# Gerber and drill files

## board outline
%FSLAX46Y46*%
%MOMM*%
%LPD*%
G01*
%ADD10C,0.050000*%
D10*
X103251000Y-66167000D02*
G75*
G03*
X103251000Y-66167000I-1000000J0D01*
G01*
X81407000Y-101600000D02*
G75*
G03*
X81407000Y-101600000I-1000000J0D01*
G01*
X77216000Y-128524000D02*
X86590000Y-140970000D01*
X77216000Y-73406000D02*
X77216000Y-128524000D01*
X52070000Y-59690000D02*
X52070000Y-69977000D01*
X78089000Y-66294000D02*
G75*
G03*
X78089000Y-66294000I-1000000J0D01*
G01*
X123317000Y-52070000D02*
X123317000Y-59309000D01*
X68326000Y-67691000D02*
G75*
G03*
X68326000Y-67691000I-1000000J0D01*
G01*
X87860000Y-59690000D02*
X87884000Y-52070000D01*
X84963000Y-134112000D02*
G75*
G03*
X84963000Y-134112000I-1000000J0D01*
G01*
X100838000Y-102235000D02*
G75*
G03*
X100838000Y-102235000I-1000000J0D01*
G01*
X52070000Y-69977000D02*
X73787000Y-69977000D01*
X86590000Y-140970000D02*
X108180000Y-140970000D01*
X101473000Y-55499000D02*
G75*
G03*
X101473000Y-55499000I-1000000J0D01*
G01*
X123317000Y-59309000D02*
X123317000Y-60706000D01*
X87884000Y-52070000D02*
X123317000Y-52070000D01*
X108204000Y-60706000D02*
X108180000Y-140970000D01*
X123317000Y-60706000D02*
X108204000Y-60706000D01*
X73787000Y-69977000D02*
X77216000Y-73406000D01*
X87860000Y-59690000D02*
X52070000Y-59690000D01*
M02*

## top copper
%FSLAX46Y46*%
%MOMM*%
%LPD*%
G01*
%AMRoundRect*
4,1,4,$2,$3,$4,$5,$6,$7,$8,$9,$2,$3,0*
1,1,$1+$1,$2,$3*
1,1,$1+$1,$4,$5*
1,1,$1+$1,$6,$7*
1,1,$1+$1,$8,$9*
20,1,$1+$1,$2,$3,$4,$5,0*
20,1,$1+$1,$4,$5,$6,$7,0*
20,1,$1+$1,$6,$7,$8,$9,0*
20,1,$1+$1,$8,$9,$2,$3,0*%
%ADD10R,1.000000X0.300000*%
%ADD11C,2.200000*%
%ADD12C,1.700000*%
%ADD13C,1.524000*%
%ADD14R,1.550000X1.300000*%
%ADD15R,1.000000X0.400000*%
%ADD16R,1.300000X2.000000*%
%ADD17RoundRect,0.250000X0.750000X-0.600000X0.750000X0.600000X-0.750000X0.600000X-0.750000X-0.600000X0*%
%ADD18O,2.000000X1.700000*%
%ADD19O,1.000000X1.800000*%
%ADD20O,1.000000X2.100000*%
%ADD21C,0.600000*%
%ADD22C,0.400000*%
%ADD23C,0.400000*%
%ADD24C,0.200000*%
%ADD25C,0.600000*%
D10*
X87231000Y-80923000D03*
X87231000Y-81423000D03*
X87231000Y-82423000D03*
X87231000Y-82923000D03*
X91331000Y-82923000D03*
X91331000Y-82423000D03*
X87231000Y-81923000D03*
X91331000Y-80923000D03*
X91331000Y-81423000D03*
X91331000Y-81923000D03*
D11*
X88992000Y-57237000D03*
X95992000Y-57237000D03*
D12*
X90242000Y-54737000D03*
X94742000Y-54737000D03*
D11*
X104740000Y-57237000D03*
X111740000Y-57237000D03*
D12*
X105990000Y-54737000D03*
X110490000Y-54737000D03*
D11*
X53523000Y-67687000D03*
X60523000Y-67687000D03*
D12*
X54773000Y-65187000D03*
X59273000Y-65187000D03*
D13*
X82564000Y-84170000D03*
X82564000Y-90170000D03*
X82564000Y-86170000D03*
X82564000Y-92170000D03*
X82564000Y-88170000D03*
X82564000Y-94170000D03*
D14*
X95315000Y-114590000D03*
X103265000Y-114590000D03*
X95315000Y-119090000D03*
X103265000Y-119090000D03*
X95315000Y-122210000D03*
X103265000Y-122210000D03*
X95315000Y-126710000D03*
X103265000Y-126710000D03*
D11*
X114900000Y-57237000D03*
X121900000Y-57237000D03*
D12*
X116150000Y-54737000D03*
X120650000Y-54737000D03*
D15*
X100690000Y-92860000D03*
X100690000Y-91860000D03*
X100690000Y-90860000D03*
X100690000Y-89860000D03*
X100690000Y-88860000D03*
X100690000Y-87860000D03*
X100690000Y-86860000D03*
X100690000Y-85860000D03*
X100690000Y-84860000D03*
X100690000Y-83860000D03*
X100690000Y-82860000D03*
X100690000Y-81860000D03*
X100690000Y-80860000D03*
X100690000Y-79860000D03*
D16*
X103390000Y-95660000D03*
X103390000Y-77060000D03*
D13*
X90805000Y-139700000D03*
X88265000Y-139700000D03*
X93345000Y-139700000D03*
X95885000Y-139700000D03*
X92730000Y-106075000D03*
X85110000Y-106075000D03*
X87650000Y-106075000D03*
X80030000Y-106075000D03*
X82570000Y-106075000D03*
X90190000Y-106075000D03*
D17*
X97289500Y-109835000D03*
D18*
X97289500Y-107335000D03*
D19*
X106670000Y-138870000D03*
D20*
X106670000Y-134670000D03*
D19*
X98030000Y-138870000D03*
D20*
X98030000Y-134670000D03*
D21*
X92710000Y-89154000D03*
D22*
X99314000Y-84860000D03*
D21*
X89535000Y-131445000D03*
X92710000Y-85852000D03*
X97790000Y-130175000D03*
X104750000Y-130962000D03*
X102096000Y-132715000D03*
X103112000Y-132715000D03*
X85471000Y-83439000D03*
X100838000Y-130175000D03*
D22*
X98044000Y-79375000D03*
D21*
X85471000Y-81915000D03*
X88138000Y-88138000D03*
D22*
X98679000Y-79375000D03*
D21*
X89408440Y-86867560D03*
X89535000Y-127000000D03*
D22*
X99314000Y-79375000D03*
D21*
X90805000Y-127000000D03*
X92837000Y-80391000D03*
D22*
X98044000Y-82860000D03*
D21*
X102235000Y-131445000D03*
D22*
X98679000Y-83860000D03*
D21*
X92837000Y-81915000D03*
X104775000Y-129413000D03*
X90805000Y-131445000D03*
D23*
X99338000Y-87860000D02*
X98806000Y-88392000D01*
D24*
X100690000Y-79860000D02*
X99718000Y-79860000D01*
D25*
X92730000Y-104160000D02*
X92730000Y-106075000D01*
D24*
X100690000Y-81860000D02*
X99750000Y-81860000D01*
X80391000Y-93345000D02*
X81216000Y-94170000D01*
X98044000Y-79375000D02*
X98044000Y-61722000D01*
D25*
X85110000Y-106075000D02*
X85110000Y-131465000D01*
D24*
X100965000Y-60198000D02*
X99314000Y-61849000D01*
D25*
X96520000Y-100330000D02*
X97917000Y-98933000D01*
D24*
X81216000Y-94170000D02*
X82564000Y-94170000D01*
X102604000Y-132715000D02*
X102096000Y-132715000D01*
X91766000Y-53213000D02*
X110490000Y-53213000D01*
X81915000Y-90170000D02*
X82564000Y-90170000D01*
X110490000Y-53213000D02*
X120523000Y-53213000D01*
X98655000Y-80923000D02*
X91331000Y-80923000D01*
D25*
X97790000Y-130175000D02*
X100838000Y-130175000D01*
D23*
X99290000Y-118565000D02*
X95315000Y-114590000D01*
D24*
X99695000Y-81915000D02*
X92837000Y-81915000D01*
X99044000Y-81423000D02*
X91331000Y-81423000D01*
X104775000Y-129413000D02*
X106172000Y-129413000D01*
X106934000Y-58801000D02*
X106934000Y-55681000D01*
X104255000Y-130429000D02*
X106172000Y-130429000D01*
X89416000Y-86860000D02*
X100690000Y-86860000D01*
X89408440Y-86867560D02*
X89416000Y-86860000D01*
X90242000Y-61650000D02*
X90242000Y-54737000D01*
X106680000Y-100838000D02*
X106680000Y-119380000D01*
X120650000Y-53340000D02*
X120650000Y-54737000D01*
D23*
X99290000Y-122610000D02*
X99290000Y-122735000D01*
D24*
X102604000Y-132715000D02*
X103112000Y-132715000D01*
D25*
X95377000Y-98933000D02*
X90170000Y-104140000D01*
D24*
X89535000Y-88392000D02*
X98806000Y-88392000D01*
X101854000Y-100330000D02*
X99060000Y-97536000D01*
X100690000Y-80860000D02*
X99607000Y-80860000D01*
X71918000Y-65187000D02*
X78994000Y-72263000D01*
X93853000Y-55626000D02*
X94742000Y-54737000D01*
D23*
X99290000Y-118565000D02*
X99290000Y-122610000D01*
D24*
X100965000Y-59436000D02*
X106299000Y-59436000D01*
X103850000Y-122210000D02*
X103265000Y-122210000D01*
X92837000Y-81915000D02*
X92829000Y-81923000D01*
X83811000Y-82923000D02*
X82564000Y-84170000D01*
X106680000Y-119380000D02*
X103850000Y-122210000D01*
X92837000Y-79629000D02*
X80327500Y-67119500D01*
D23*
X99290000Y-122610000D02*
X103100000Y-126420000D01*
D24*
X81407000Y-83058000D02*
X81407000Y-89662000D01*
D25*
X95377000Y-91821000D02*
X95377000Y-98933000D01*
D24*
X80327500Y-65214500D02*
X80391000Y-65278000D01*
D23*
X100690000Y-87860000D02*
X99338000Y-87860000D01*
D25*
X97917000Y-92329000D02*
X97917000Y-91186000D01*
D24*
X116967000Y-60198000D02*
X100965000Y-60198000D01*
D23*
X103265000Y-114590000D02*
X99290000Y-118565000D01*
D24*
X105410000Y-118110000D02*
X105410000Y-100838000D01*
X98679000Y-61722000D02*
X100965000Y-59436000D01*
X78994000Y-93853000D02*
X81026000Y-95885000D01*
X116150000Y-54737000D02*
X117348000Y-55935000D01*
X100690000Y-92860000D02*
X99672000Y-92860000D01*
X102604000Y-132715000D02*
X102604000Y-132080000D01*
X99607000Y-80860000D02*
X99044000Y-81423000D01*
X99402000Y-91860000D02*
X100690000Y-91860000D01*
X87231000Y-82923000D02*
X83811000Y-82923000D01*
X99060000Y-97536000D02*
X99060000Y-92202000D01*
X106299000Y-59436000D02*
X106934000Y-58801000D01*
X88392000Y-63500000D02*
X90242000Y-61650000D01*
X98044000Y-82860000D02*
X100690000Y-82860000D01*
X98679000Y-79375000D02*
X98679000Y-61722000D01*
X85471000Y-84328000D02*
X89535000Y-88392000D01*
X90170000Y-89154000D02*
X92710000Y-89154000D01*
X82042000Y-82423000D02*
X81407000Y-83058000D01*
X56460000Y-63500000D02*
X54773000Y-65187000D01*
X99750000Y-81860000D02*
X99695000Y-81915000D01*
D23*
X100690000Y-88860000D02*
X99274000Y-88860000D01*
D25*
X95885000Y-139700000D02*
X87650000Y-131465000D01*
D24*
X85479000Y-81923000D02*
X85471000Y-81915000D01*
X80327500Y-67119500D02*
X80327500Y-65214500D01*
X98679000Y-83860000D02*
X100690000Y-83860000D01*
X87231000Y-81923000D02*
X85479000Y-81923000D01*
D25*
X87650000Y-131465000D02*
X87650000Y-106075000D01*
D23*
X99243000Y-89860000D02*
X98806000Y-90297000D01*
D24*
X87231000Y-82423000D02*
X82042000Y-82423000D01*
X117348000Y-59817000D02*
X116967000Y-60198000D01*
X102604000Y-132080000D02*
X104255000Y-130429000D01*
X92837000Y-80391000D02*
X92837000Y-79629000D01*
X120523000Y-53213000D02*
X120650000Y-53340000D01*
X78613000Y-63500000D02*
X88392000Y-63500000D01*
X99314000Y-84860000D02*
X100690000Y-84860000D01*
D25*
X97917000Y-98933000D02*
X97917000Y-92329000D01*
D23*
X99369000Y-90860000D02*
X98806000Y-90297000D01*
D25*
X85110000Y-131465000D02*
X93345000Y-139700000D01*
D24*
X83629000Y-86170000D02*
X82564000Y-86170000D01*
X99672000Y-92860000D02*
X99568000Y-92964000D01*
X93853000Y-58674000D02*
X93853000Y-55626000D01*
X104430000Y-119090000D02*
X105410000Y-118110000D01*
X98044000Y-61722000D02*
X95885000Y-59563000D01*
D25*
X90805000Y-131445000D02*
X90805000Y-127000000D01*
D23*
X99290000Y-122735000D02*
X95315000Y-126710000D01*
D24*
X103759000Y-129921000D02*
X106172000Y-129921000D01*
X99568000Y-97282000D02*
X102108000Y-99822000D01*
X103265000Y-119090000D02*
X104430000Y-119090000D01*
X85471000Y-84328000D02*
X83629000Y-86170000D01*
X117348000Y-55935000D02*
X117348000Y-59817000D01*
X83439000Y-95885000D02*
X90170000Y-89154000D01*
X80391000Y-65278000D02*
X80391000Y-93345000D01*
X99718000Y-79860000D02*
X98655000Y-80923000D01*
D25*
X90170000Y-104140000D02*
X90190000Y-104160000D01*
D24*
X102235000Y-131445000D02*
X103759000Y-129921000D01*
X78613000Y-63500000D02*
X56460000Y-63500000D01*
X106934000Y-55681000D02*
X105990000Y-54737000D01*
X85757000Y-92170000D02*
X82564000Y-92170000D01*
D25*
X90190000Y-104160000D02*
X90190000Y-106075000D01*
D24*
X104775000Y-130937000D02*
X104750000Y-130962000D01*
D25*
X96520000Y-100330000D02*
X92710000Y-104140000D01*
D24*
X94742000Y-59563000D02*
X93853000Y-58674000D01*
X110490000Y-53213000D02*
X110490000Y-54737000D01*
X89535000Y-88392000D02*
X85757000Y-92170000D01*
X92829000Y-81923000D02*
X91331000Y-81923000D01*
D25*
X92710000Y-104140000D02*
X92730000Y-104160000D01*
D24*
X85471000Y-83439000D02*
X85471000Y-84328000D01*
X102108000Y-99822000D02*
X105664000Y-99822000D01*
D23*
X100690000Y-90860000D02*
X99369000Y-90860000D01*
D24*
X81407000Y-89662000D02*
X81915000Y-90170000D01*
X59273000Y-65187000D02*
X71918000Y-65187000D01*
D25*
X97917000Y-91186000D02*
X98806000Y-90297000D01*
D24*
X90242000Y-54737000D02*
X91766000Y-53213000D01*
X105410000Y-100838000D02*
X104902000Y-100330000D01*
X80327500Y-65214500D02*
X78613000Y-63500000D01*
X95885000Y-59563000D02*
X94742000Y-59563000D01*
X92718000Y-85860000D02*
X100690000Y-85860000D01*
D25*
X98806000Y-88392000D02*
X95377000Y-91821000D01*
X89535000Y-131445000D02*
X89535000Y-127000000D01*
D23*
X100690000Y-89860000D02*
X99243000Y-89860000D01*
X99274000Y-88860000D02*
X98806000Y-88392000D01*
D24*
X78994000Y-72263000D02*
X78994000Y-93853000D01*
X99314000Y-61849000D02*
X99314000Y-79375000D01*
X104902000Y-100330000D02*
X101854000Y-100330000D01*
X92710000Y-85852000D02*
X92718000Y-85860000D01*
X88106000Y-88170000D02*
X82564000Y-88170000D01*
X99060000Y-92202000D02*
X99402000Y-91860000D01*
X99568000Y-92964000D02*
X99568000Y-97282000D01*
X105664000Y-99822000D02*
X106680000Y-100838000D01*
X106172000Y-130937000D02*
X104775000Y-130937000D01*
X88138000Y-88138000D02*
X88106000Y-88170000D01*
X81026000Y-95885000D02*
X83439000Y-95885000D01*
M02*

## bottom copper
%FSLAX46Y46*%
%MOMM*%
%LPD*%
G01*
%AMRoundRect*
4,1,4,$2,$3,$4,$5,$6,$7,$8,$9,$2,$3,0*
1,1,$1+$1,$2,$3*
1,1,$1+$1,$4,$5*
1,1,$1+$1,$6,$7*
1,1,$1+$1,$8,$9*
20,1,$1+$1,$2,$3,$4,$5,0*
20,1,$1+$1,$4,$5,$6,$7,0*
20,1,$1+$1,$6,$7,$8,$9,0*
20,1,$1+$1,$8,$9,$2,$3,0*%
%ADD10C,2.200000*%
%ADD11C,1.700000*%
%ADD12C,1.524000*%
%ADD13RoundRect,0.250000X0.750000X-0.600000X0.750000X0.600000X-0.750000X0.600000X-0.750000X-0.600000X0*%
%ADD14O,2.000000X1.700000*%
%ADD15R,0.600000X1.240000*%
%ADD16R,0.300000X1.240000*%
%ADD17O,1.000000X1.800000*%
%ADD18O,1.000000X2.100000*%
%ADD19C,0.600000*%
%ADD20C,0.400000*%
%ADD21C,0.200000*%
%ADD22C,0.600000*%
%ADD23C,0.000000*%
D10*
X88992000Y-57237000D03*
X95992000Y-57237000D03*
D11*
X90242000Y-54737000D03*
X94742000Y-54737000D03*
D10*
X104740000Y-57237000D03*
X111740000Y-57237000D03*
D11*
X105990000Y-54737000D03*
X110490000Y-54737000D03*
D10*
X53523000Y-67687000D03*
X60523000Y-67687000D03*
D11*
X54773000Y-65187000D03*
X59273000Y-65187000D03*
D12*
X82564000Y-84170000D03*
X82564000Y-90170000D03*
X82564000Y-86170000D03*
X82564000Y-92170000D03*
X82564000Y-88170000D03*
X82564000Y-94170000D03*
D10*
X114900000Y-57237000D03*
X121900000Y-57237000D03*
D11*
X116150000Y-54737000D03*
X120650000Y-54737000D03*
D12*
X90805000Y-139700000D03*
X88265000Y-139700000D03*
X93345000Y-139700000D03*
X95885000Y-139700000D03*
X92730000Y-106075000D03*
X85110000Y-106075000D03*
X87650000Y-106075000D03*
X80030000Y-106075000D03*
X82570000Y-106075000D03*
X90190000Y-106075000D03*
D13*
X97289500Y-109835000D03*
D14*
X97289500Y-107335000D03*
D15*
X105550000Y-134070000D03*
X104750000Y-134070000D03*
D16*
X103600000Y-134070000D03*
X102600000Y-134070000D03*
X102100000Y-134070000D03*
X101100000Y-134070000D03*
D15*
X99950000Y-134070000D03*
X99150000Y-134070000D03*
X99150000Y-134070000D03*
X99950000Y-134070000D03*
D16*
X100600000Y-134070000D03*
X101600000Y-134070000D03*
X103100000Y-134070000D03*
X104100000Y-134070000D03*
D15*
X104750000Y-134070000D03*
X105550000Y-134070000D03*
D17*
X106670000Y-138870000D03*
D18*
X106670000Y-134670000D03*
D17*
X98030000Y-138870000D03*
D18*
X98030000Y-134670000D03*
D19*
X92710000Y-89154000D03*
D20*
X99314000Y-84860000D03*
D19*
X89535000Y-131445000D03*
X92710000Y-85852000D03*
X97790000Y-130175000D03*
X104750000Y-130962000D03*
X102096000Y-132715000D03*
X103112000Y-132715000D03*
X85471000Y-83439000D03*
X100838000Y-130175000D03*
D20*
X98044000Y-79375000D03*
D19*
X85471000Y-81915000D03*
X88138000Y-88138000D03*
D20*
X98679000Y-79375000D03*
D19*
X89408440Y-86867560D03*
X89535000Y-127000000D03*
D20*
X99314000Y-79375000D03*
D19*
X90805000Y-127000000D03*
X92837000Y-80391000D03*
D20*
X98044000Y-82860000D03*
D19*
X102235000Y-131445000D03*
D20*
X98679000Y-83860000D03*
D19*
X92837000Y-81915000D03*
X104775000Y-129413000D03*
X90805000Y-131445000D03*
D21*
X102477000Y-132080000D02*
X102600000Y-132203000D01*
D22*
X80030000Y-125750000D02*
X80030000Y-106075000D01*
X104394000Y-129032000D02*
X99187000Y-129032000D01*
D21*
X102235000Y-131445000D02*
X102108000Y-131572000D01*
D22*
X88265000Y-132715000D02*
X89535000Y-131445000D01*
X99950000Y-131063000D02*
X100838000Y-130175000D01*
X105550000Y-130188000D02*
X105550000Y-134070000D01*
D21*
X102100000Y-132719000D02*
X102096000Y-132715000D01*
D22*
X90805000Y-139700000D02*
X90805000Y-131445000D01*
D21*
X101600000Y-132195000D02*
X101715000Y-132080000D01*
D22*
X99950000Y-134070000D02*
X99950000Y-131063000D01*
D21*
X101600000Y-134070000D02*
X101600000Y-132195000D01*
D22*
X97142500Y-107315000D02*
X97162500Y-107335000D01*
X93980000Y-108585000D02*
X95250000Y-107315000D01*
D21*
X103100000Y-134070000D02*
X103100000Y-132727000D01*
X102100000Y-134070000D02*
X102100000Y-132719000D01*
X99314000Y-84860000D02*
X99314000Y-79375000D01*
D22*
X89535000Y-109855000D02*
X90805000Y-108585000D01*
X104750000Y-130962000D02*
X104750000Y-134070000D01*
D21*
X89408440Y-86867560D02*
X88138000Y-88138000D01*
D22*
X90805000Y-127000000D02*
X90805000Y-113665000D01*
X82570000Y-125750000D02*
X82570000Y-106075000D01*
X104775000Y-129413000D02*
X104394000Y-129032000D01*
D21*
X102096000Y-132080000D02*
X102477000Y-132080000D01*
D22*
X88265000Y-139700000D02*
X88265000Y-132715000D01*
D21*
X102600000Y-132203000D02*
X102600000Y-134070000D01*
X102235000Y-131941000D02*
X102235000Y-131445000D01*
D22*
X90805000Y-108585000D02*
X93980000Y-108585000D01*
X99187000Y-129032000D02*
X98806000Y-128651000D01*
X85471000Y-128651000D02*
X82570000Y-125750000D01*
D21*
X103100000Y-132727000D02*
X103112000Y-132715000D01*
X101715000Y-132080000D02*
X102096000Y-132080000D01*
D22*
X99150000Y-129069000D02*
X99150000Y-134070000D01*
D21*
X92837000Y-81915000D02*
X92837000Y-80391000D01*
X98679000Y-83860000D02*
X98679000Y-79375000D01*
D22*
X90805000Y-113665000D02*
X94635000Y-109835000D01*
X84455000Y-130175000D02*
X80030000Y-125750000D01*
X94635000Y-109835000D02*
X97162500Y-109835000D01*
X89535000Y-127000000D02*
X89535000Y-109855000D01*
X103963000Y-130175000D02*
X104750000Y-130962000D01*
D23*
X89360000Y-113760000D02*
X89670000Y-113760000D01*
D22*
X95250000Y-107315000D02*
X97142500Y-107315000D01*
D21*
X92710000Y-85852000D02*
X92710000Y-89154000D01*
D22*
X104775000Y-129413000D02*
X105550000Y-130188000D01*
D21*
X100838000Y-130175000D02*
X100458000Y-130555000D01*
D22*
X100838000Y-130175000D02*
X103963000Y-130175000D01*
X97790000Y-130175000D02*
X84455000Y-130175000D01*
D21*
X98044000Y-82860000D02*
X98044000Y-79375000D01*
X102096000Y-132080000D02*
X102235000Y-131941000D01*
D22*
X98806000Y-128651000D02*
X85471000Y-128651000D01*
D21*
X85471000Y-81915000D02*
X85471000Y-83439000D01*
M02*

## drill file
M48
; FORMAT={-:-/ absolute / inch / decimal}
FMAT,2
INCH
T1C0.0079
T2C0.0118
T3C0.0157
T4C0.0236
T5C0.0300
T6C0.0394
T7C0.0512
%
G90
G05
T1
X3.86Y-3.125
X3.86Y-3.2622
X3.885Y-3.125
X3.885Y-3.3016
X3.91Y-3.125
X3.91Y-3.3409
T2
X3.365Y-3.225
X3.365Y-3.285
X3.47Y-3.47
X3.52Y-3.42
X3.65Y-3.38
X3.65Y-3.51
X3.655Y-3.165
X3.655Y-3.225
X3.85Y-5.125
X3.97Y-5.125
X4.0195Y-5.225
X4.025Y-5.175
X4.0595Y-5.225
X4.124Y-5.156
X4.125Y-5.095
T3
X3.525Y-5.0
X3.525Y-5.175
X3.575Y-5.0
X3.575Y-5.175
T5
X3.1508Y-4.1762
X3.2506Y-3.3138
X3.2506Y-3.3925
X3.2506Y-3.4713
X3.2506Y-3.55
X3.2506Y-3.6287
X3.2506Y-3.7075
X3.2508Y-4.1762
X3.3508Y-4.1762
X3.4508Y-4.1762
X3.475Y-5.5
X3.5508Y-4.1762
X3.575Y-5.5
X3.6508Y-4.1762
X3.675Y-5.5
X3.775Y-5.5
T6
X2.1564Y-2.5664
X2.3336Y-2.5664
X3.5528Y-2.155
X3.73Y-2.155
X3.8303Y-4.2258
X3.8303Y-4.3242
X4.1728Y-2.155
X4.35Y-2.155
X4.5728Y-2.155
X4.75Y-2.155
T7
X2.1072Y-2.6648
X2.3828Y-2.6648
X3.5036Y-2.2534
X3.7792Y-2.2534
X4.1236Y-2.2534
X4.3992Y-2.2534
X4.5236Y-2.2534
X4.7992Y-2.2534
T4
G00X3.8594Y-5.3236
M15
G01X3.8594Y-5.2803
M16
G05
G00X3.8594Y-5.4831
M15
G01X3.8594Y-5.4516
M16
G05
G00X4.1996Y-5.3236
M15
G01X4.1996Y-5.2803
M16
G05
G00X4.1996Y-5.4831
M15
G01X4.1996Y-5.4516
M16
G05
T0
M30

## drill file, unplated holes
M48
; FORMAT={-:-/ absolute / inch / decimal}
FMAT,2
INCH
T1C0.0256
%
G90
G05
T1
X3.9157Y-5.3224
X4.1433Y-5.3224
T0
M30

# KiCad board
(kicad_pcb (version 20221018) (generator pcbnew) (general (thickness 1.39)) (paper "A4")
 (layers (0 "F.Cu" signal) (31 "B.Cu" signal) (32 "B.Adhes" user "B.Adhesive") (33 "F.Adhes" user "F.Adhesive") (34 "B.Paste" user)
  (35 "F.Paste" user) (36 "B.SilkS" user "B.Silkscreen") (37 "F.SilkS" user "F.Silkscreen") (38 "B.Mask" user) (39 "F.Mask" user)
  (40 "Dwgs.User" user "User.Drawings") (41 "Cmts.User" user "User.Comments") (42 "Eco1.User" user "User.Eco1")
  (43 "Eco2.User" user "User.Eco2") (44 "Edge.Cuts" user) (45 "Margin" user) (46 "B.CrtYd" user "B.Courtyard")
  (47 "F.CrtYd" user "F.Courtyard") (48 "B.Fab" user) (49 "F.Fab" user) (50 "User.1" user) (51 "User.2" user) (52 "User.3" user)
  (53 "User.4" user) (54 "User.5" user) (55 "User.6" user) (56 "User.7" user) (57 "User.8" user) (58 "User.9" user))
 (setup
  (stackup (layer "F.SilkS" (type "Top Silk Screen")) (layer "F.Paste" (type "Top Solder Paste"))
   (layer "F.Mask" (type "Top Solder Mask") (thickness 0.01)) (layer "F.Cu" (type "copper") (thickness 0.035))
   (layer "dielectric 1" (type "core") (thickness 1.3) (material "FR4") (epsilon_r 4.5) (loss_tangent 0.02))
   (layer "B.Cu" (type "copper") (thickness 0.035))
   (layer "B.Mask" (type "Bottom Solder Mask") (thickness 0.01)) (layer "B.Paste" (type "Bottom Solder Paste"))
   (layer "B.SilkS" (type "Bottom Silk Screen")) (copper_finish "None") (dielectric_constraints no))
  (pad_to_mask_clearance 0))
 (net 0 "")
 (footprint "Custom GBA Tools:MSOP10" (layer "F.Cu") (at 89.281 81.923 -90)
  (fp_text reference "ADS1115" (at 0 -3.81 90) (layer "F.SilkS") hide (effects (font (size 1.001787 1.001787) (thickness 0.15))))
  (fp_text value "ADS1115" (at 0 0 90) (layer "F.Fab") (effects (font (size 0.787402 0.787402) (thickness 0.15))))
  (pad "1" smd rect (at -1 2.05 270) (size 0.3 1) (layers "F.Cu"))
  (pad "2" smd rect (at -0.5 2.05 270) (size 0.3 1) (layers "F.Cu"))
  (pad "A0" smd rect (at 0.5 2.05 270) (size 0.3 1) (layers "F.Cu"))
  (pad "A1" smd rect (at 1 2.05 270) (size 0.3 1) (layers "F.Cu"))
  (pad "A2" smd rect (at 1 -2.05 270) (size 0.3 1) (layers "F.Cu"))
  (pad "A3" smd rect (at 0.5 -2.05 270) (size 0.3 1) (layers "F.Cu"))
  (pad "GND" smd rect (at 0 2.05 270) (size 0.3 1) (layers "F.Cu"))
  (pad "SCL" smd rect (at -1 -2.05 270) (size 0.3 1) (layers "F.Cu"))
  (pad "SDA" smd rect (at -0.5 -2.05 270) (size 0.3 1) (layers "F.Cu"))
  (pad "VDD" smd rect (at 0 -2.05 270) (size 0.3 1) (layers "F.Cu")))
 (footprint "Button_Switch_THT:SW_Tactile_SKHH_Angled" (layer "F.Cu") (at 90.242 54.737)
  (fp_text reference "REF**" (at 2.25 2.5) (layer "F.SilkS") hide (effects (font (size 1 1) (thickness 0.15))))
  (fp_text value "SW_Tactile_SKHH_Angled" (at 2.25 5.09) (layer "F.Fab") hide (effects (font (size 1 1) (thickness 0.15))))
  (pad "" thru_hole circle (at -1.25 2.5 180) (size 2.2 2.2) (drill 1.3) (layers "*.Cu" "*.Mask"))
  (pad "" thru_hole circle (at 5.75 2.5 180) (size 2.2 2.2) (drill 1.3) (layers "*.Cu" "*.Mask"))
  (pad "1" thru_hole circle (at 0 0 180) (size 1.7 1.7) (drill 1) (layers "*.Cu" "*.Mask"))
  (pad "2" thru_hole circle (at 4.5 0 180) (size 1.7 1.7) (drill 1) (layers "*.Cu" "*.Mask")))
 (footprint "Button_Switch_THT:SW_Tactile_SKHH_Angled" (layer "F.Cu") (at 105.99 54.737)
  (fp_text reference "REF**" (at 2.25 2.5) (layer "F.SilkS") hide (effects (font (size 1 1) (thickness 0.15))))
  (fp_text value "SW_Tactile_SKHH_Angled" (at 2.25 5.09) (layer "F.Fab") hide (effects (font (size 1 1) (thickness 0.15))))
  (pad "" thru_hole circle (at -1.25 2.5 180) (size 2.2 2.2) (drill 1.3) (layers "*.Cu" "*.Mask"))
  (pad "" thru_hole circle (at 5.75 2.5 180) (size 2.2 2.2) (drill 1.3) (layers "*.Cu" "*.Mask"))
  (pad "1" thru_hole circle (at 0 0 180) (size 1.7 1.7) (drill 1) (layers "*.Cu" "*.Mask"))
  (pad "2" thru_hole circle (at 4.5 0 180) (size 1.7 1.7) (drill 1) (layers "*.Cu" "*.Mask")))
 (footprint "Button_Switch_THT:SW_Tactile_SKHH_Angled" (layer "F.Cu") (at 54.773 65.187)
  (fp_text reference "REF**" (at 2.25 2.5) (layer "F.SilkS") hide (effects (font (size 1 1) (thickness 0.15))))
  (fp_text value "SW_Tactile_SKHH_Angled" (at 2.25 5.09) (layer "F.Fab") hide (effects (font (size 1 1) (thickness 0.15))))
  (pad "" thru_hole circle (at -1.25 2.5 180) (size 2.2 2.2) (drill 1.3) (layers "*.Cu" "*.Mask"))
  (pad "" thru_hole circle (at 5.75 2.5 180) (size 2.2 2.2) (drill 1.3) (layers "*.Cu" "*.Mask"))
  (pad "1" thru_hole circle (at 0 0 180) (size 1.7 1.7) (drill 1) (layers "*.Cu" "*.Mask"))
  (pad "2" thru_hole circle (at 4.5 0 180) (size 1.7 1.7) (drill 1) (layers "*.Cu" "*.Mask")))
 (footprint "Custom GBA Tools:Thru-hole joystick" (layer "F.Cu") (at 69.964 92.97)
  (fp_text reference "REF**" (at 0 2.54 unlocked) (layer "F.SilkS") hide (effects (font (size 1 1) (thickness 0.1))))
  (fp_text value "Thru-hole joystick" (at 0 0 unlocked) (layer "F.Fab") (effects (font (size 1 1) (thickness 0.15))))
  (pad "A1" thru_hole circle (at 12.6 -8.8) (size 1.524 1.524) (drill 0.762) (layers "*.Cu" "*.Mask"))
  (pad "A2" thru_hole circle (at 12.6 -2.8) (size 1.524 1.524) (drill 0.762) (layers "*.Cu" "*.Mask"))
  (pad "GND" thru_hole circle (at 12.6 -6.8) (size 1.524 1.524) (drill 0.762) (layers "*.Cu" "*.Mask"))
  (pad "GND" thru_hole circle (at 12.6 -0.8) (size 1.524 1.524) (drill 0.762) (layers "*.Cu" "*.Mask"))
  (pad "SW" thru_hole circle (at 12.6 -4.8) (size 1.524 1.524) (drill 0.762) (layers "*.Cu" "*.Mask"))
  (pad "VCC" thru_hole circle (at 12.6 1.2) (size 1.524 1.524) (drill 0.762) (layers "*.Cu" "*.Mask")))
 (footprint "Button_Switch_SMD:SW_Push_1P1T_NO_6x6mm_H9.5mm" (layer "F.Cu") (at 99.29 116.84)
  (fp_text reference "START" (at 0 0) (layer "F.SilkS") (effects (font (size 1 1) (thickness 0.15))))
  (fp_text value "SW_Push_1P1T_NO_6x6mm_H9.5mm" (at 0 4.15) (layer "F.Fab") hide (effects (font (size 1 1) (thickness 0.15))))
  (pad "1" smd rect (at -3.975 -2.25) (size 1.55 1.3) (layers "F.Cu" "F.Paste" "F.Mask"))
  (pad "1" smd rect (at 3.975 -2.25) (size 1.55 1.3) (layers "F.Cu" "F.Paste" "F.Mask"))
  (pad "2" smd rect (at -3.975 2.25) (size 1.55 1.3) (layers "F.Cu" "F.Paste" "F.Mask"))
  (pad "2" smd rect (at 3.975 2.25) (size 1.55 1.3) (layers "F.Cu" "F.Paste" "F.Mask")))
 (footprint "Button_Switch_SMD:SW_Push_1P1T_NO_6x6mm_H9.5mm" (layer "F.Cu") (at 99.29 124.46)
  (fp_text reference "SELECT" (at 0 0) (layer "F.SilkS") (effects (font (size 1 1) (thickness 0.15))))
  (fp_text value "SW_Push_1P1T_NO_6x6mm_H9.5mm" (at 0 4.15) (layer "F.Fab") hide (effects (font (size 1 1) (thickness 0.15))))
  (pad "1" smd rect (at -3.975 -2.25) (size 1.55 1.3) (layers "F.Cu" "F.Paste" "F.Mask"))
  (pad "1" smd rect (at 3.975 -2.25) (size 1.55 1.3) (layers "F.Cu" "F.Paste" "F.Mask"))
  (pad "2" smd rect (at -3.975 2.25) (size 1.55 1.3) (layers "F.Cu" "F.Paste" "F.Mask"))
  (pad "2" smd rect (at 3.975 2.25) (size 1.55 1.3) (layers "F.Cu" "F.Paste" "F.Mask")))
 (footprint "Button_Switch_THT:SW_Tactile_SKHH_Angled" (layer "F.Cu") (at 116.15 54.737)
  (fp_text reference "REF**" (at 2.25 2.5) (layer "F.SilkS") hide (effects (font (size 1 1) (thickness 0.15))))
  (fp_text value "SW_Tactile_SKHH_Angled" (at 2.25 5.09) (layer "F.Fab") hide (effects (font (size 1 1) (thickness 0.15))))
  (pad "" thru_hole circle (at -1.25 2.5 180) (size 2.2 2.2) (drill 1.3) (layers "*.Cu" "*.Mask"))
  (pad "" thru_hole circle (at 5.75 2.5 180) (size 2.2 2.2) (drill 1.3) (layers "*.Cu" "*.Mask"))
  (pad "1" thru_hole circle (at 0 0 180) (size 1.7 1.7) (drill 1) (layers "*.Cu" "*.Mask"))
  (pad "2" thru_hole circle (at 4.5 0 180) (size 1.7 1.7) (drill 1) (layers "*.Cu" "*.Mask")))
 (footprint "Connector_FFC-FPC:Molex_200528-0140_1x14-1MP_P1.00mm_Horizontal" (layer "F.Cu") (at 101.6 86.36 90)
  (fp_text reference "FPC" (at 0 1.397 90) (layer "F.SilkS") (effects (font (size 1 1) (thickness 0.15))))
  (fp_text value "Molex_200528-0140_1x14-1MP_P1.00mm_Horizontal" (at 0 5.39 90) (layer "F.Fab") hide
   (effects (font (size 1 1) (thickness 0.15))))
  (pad "1" smd rect (at -6.5 -0.91 90) (size 0.4 1) (layers "F.Cu" "F.Paste" "F.Mask"))
  (pad "2" smd rect (at -5.5 -0.91 90) (size 0.4 1) (layers "F.Cu" "F.Paste" "F.Mask"))
  (pad "3" smd rect (at -4.5 -0.91 90) (size 0.4 1) (layers "F.Cu" "F.Paste" "F.Mask"))
  (pad "4" smd rect (at -3.5 -0.91 90) (size 0.4 1) (layers "F.Cu" "F.Paste" "F.Mask"))
  (pad "5" smd rect (at -2.5 -0.91 90) (size 0.4 1) (layers "F.Cu" "F.Paste" "F.Mask"))
  (pad "6" smd rect (at -1.5 -0.91 90) (size 0.4 1) (layers "F.Cu" "F.Paste" "F.Mask"))
  (pad "7" smd rect (at -0.5 -0.91 90) (size 0.4 1) (layers "F.Cu" "F.Paste" "F.Mask"))
  (pad "8" smd rect (at 0.5 -0.91 90) (size 0.4 1) (layers "F.Cu" "F.Paste" "F.Mask"))
  (pad "9" smd rect (at 1.5 -0.91 90) (size 0.4 1) (layers "F.Cu" "F.Paste" "F.Mask"))
  (pad "10" smd rect (at 2.5 -0.91 90) (size 0.4 1) (layers "F.Cu" "F.Paste" "F.Mask"))
  (pad "11" smd rect (at 3.5 -0.91 90) (size 0.4 1) (layers "F.Cu" "F.Paste" "F.Mask"))
  (pad "12" smd rect (at 4.5 -0.91 90) (size 0.4 1) (layers "F.Cu" "F.Paste" "F.Mask"))
  (pad "13" smd rect (at 5.5 -0.91 90) (size 0.4 1) (layers "F.Cu" "F.Paste" "F.Mask"))
  (pad "14" smd rect (at 6.5 -0.91 90) (size 0.4 1) (layers "F.Cu" "F.Paste" "F.Mask"))
  (pad "MP" smd rect (at -9.3 1.79 90) (size 2 1.3) (layers "F.Cu" "F.Paste" "F.Mask"))
  (pad "MP" smd rect (at 9.3 1.79 90) (size 2 1.3) (layers "F.Cu" "F.Paste" "F.Mask")))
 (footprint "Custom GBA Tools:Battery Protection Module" (layer "B.Cu") (at 97.155 140.97 180)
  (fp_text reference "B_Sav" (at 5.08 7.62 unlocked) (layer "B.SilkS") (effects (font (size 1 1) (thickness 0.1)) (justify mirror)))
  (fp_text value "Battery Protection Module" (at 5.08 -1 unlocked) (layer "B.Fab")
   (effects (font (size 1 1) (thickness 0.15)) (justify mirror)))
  (pad "B+" thru_hole circle (at 6.35 1.27 180) (size 1.524 1.524) (drill 0.762) (layers "*.Cu" "*.Mask"))
  (pad "B-" thru_hole circle (at 8.89 1.27 180) (size 1.524 1.524) (drill 0.762) (layers "*.Cu" "*.Mask"))
  (pad "P+" thru_hole circle (at 3.81 1.27 180) (size 1.524 1.524) (drill 0.762) (layers "*.Cu" "*.Mask"))
  (pad "P-" thru_hole circle (at 1.27 1.27 180) (size 1.524 1.524) (drill 0.762) (layers "*.Cu" "*.Mask")))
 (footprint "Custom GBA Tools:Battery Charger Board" (layer "B.Cu") (at 78.76 104.805)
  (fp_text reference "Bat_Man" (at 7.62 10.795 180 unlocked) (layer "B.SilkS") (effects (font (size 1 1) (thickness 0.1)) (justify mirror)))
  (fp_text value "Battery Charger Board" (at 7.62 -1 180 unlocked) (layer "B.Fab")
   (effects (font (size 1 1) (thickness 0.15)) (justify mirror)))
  (pad "5V" thru_hole circle (at 13.97 1.27) (size 1.524 1.524) (drill 0.762) (layers "*.Cu" "*.Mask"))
  (pad "Bat+" thru_hole circle (at 6.35 1.27) (size 1.524 1.524) (drill 0.762) (layers "*.Cu" "*.Mask"))
  (pad "Bat-" thru_hole circle (at 8.89 1.27) (size 1.524 1.524) (drill 0.762) (layers "*.Cu" "*.Mask"))
  (pad "CHG+" thru_hole circle (at 1.27 1.27) (size 1.524 1.524) (drill 0.762) (layers "*.Cu" "*.Mask"))
  (pad "CHG-" thru_hole circle (at 3.81 1.27) (size 1.524 1.524) (drill 0.762) (layers "*.Cu" "*.Mask"))
  (pad "GND" thru_hole circle (at 11.43 1.27) (size 1.524 1.524) (drill 0.762) (layers "*.Cu" "*.Mask")))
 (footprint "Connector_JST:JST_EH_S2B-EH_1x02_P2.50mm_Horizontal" (layer "B.Cu") (at 97.2895 109.835 90)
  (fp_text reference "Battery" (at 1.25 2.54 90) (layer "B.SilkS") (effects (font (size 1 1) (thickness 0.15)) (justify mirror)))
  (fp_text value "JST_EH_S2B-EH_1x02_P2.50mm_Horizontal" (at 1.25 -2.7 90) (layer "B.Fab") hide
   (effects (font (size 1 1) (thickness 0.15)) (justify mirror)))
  (pad "1" thru_hole roundrect (at 0 0 90) (size 1.7 2) (drill 1) (layers "*.Cu" "*.Mask") (roundrect_rratio 0.1470588235))
  (pad "2" thru_hole oval (at 2.5 0 90) (size 1.7 2) (drill 1) (layers "*.Cu" "*.Mask")))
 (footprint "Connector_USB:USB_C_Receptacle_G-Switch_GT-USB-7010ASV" (layer "B.Cu") (at 102.35 137.795 180)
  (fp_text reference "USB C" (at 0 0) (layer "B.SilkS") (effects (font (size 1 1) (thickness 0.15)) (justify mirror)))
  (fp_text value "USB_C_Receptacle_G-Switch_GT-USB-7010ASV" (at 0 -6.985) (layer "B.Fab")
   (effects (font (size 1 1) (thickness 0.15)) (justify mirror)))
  (pad "" np_thru_hole circle (at -2.89 2.605 180) (size 0.65 0.65) (drill 0.65) (layers "*.Cu" "*.Mask"))
  (pad "" np_thru_hole circle (at 2.89 2.605 180) (size 0.65 0.65) (drill 0.65) (layers "*.Cu" "*.Mask"))
  (pad "A1" smd rect (at -3.2 3.725 180) (size 0.6 1.24) (layers "B.Cu" "B.Paste" "B.Mask"))
  (pad "A4" smd rect (at -2.4 3.725 180) (size 0.6 1.24) (layers "B.Cu" "B.Paste" "B.Mask"))
  (pad "A5" smd rect (at -1.25 3.725 180) (size 0.3 1.24) (layers "B.Cu" "B.Paste" "B.Mask"))
  (pad "A6" smd rect (at -0.25 3.725 180) (size 0.3 1.24) (layers "B.Cu" "B.Paste" "B.Mask"))
  (pad "A7" smd rect (at 0.25 3.725 180) (size 0.3 1.24) (layers "B.Cu" "B.Paste" "B.Mask"))
  (pad "A8" smd rect (at 1.25 3.725 180) (size 0.3 1.24) (layers "B.Cu" "B.Paste" "B.Mask"))
  (pad "A9" smd rect (at 2.4 3.725 180) (size 0.6 1.24) (layers "B.Cu" "B.Paste" "B.Mask"))
  (pad "A12" smd rect (at 3.2 3.725 180) (size 0.6 1.24) (layers "B.Cu" "B.Paste" "B.Mask"))
  (pad "B1" smd rect (at 3.2 3.725 180) (size 0.6 1.24) (layers "B.Cu" "B.Paste" "B.Mask"))
  (pad "B4" smd rect (at 2.4 3.725 180) (size 0.6 1.24) (layers "B.Cu" "B.Paste" "B.Mask"))
  (pad "B5" smd rect (at 1.75 3.725 180) (size 0.3 1.24) (layers "B.Cu" "B.Paste" "B.Mask"))
  (pad "B6" smd rect (at 0.75 3.725 180) (size 0.3 1.24) (layers "B.Cu" "B.Paste" "B.Mask"))
  (pad "B7" smd rect (at -0.75 3.725 180) (size 0.3 1.24) (layers "B.Cu" "B.Paste" "B.Mask"))
  (pad "B8" smd rect (at -1.75 3.725 180) (size 0.3 1.24) (layers "B.Cu" "B.Paste" "B.Mask"))
  (pad "B9" smd rect (at -2.4 3.725 180) (size 0.6 1.24) (layers "B.Cu" "B.Paste" "B.Mask"))
  (pad "B12" smd rect (at -3.2 3.725 180) (size 0.6 1.24) (layers "B.Cu" "B.Paste" "B.Mask"))
  (pad "S1" thru_hole oval (at -4.32 -1.075 180) (size 1 1.8) (drill oval 0.6 1.4) (layers "*.Cu" "*.Mask"))
  (pad "S1" thru_hole oval (at -4.32 3.125 180) (size 1 2.1) (drill oval 0.6 1.7) (layers "*.Cu" "*.Mask"))
  (pad "S1" thru_hole oval (at 4.32 -1.075 180) (size 1 1.8) (drill oval 0.6 1.4) (layers "*.Cu" "*.Mask"))
  (pad "S1" thru_hole oval (at 4.32 3.125 180) (size 1 2.1) (drill oval 0.6 1.7) (layers "*.Cu" "*.Mask")))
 (gr_circle (center 102.251 66.167) (end 103.251 66.167) (stroke (width 0.05) (type default)) (fill none) (layer "Edge.Cuts"))
 (gr_circle (center 80.407 101.6) (end 81.407 101.6) (stroke (width 0.05) (type default)) (fill none) (layer "Edge.Cuts"))
 (gr_line (start 77.216 128.524) (end 86.59 140.97) (stroke (width 0.05) (type default)) (layer "Edge.Cuts"))
 (gr_line (start 77.216 73.406) (end 77.216 128.524) (stroke (width 0.05) (type default)) (layer "Edge.Cuts"))
 (gr_line (start 52.07 59.69) (end 52.07 69.977) (stroke (width 0.05) (type default)) (layer "Edge.Cuts"))
 (gr_circle (center 77.089 66.294) (end 78.089 66.294) (stroke (width 0.05) (type default)) (fill none) (layer "Edge.Cuts"))
 (gr_line (start 123.317 52.07) (end 123.317 59.309) (stroke (width 0.05) (type default)) (layer "Edge.Cuts"))
 (gr_circle (center 67.326 67.691) (end 68.326 67.691) (stroke (width 0.05) (type default)) (fill none) (layer "Edge.Cuts"))
 (gr_line (start 87.86 59.69) (end 87.884 52.07) (stroke (width 0.05) (type default)) (layer "Edge.Cuts"))
 (gr_circle (center 83.963 134.112) (end 84.963 134.112) (stroke (width 0.05) (type default)) (fill none) (layer "Edge.Cuts"))
 (gr_circle (center 99.838 102.235) (end 100.838 102.235) (stroke (width 0.05) (type default)) (fill none) (layer "Edge.Cuts"))
 (gr_line (start 52.07 69.977) (end 73.787 69.977) (stroke (width 0.05) (type default)) (layer "Edge.Cuts"))
 (gr_line (start 86.59 140.97) (end 108.18 140.97) (stroke (width 0.05) (type default)) (layer "Edge.Cuts"))
 (gr_circle (center 100.473 55.499) (end 101.473 55.499) (stroke (width 0.05) (type default)) (fill none) (layer "Edge.Cuts"))
 (gr_line (start 123.317 59.309) (end 123.317 60.706) (stroke (width 0.05) (type default)) (layer "Edge.Cuts"))
 (gr_line (start 87.884 52.07) (end 123.317 52.07) (stroke (width 0.05) (type default)) (layer "Edge.Cuts"))
 (gr_line (start 108.204 60.706) (end 108.18 140.97) (stroke (width 0.05) (type default)) (layer "Edge.Cuts"))
 (gr_line (start 123.317 60.706) (end 108.204 60.706) (stroke (width 0.05) (type default)) (layer "Edge.Cuts"))
 (gr_line (start 73.787 69.977) (end 77.216 73.406) (stroke (width 0.05) (type default)) (layer "Edge.Cuts"))
 (gr_line (start 87.86 59.69) (end 52.07 59.69) (stroke (width 0.05) (type default)) (layer "Edge.Cuts"))
 (segment (start 99.338 87.86) (end 98.806 88.392) (width 0.4) (layer "F.Cu") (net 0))
 (segment (start 100.69 79.86) (end 99.718 79.86) (width 0.2) (layer "F.Cu") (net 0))
 (segment (start 92.73 104.16) (end 92.73 106.075) (width 0.6) (layer "F.Cu") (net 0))
 (segment (start 100.69 81.86) (end 99.75 81.86) (width 0.2) (layer "F.Cu") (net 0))
 (segment (start 80.391 93.345) (end 81.216 94.17) (width 0.2) (layer "F.Cu") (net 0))
 (segment (start 98.044 79.375) (end 98.044 61.722) (width 0.2) (layer "F.Cu") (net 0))
 (segment (start 85.11 106.075) (end 85.11 131.465) (width 0.6) (layer "F.Cu") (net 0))
 (segment (start 100.965 60.198) (end 99.314 61.849) (width 0.2) (layer "F.Cu") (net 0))
 (segment (start 96.52 100.33) (end 97.917 98.933) (width 0.6) (layer "F.Cu") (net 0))
 (segment (start 81.216 94.17) (end 82.564 94.17) (width 0.2) (layer "F.Cu") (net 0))
 (segment (start 102.604 132.715) (end 102.096 132.715) (width 0.2) (layer "F.Cu") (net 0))
 (segment (start 91.766 53.213) (end 110.49 53.213) (width 0.2) (layer "F.Cu") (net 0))
 (segment (start 81.915 90.17) (end 82.564 90.17) (width 0.2) (layer "F.Cu") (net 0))
 (segment (start 110.49 53.213) (end 120.523 53.213) (width 0.2) (layer "F.Cu") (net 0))
 (segment (start 98.655 80.923) (end 91.331 80.923) (width 0.2) (layer "F.Cu") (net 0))
 (segment (start 97.79 130.175) (end 100.838 130.175) (width 0.6) (layer "F.Cu") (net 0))
 (segment (start 99.29 118.565) (end 95.315 114.59) (width 0.4) (layer "F.Cu") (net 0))
 (segment (start 99.695 81.915) (end 92.837 81.915) (width 0.2) (layer "F.Cu") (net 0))
 (segment (start 99.044 81.423) (end 91.331 81.423) (width 0.2) (layer "F.Cu") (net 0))
 (segment (start 104.775 129.413) (end 106.172 129.413) (width 0.2) (layer "F.Cu") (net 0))
 (segment (start 106.934 58.801) (end 106.934 55.681) (width 0.2) (layer "F.Cu") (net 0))
 (segment (start 104.255 130.429) (end 106.172 130.429) (width 0.2) (layer "F.Cu") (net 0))
 (segment (start 89.416 86.86) (end 100.69 86.86) (width 0.2) (layer "F.Cu") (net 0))
 (segment (start 89.40844 86.86756) (end 89.416 86.86) (width 0.2) (layer "F.Cu") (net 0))
 (segment (start 90.242 61.65) (end 90.242 54.737) (width 0.2) (layer "F.Cu") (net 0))
 (segment (start 106.68 100.838) (end 106.68 119.38) (width 0.2) (layer "F.Cu") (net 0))
 (segment (start 120.65 53.34) (end 120.65 54.737) (width 0.2) (layer "F.Cu") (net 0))
 (segment (start 99.29 122.61) (end 99.29 122.735) (width 0.4) (layer "F.Cu") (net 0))
 (segment (start 102.604 132.715) (end 103.112 132.715) (width 0.2) (layer "F.Cu") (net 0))
 (segment (start 95.377 98.933) (end 90.17 104.14) (width 0.6) (layer "F.Cu") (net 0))
 (segment (start 89.535 88.392) (end 98.806 88.392) (width 0.2) (layer "F.Cu") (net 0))
 (segment (start 101.854 100.33) (end 99.06 97.536) (width 0.2) (layer "F.Cu") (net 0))
 (segment (start 100.69 80.86) (end 99.607 80.86) (width 0.2) (layer "F.Cu") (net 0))
 (segment (start 71.918 65.187) (end 78.994 72.263) (width 0.2) (layer "F.Cu") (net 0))
 (segment (start 93.853 55.626) (end 94.742 54.737) (width 0.2) (layer "F.Cu") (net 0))
 (segment (start 99.29 118.565) (end 99.29 122.61) (width 0.4) (layer "F.Cu") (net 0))
 (segment (start 100.965 59.436) (end 106.299 59.436) (width 0.2) (layer "F.Cu") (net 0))
 (segment (start 103.85 122.21) (end 103.265 122.21) (width 0.2) (layer "F.Cu") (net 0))
 (segment (start 92.837 81.915) (end 92.829 81.923) (width 0.2) (layer "F.Cu") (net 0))
 (segment (start 83.811 82.923) (end 82.564 84.17) (width 0.2) (layer "F.Cu") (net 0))
 (segment (start 106.68 119.38) (end 103.85 122.21) (width 0.2) (layer "F.Cu") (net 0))
 (segment (start 92.837 79.629) (end 80.3275 67.1195) (width 0.2) (layer "F.Cu") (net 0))
 (segment (start 99.29 122.61) (end 103.1 126.42) (width 0.4) (layer "F.Cu") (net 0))
 (segment (start 81.407 83.058) (end 81.407 89.662) (width 0.2) (layer "F.Cu") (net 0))
 (segment (start 95.377 91.821) (end 95.377 98.933) (width 0.6) (layer "F.Cu") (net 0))
 (segment (start 80.3275 65.2145) (end 80.391 65.278) (width 0.2) (layer "F.Cu") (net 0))
 (segment (start 100.69 87.86) (end 99.338 87.86) (width 0.4) (layer "F.Cu") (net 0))
 (segment (start 97.917 92.329) (end 97.917 91.186) (width 0.6) (layer "F.Cu") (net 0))
 (segment (start 116.967 60.198) (end 100.965 60.198) (width 0.2) (layer "F.Cu") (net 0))
 (segment (start 103.265 114.59) (end 99.29 118.565) (width 0.4) (layer "F.Cu") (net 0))
 (segment (start 105.41 118.11) (end 105.41 100.838) (width 0.2) (layer "F.Cu") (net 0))
 (segment (start 98.679 61.722) (end 100.965 59.436) (width 0.2) (layer "F.Cu") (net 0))
 (segment (start 78.994 93.853) (end 81.026 95.885) (width 0.2) (layer "F.Cu") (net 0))
 (segment (start 116.15 54.737) (end 117.348 55.935) (width 0.2) (layer "F.Cu") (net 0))
 (segment (start 100.69 92.86) (end 99.672 92.86) (width 0.2) (layer "F.Cu") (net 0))
 (segment (start 102.604 132.715) (end 102.604 132.08) (width 0.2) (layer "F.Cu") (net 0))
 (segment (start 99.607 80.86) (end 99.044 81.423) (width 0.2) (layer "F.Cu") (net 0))
 (segment (start 99.402 91.86) (end 100.69 91.86) (width 0.2) (layer "F.Cu") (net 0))
 (segment (start 87.231 82.923) (end 83.811 82.923) (width 0.2) (layer "F.Cu") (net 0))
 (segment (start 99.06 97.536) (end 99.06 92.202) (width 0.2) (layer "F.Cu") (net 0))
 (segment (start 106.299 59.436) (end 106.934 58.801) (width 0.2) (layer "F.Cu") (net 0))
 (segment (start 88.392 63.5) (end 90.242 61.65) (width 0.2) (layer "F.Cu") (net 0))
 (segment (start 98.044 82.86) (end 100.69 82.86) (width 0.2) (layer "F.Cu") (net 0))
 (segment (start 98.679 79.375) (end 98.679 61.722) (width 0.2) (layer "F.Cu") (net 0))
 (segment (start 85.471 84.328) (end 89.535 88.392) (width 0.2) (layer "F.Cu") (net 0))
 (segment (start 90.17 89.154) (end 92.71 89.154) (width 0.2) (layer "F.Cu") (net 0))
 (segment (start 82.042 82.423) (end 81.407 83.058) (width 0.2) (layer "F.Cu") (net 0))
 (segment (start 56.46 63.5) (end 54.773 65.187) (width 0.2) (layer "F.Cu") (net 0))
 (segment (start 99.75 81.86) (end 99.695 81.915) (width 0.2) (layer "F.Cu") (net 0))
 (segment (start 100.69 88.86) (end 99.274 88.86) (width 0.4) (layer "F.Cu") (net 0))
 (segment (start 95.885 139.7) (end 87.65 131.465) (width 0.6) (layer "F.Cu") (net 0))
 (segment (start 85.479 81.923) (end 85.471 81.915) (width 0.2) (layer "F.Cu") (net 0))
 (segment (start 80.3275 67.1195) (end 80.3275 65.2145) (width 0.2) (layer "F.Cu") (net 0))
 (segment (start 98.679 83.86) (end 100.69 83.86) (width 0.2) (layer "F.Cu") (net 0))
 (segment (start 87.231 81.923) (end 85.479 81.923) (width 0.2) (layer "F.Cu") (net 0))
 (segment (start 87.65 131.465) (end 87.65 106.075) (width 0.6) (layer "F.Cu") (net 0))
 (segment (start 99.243 89.86) (end 98.806 90.297) (width 0.4) (layer "F.Cu") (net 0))
 (segment (start 87.231 82.423) (end 82.042 82.423) (width 0.2) (layer "F.Cu") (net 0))
 (segment (start 117.348 59.817) (end 116.967 60.198) (width 0.2) (layer "F.Cu") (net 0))
 (segment (start 102.604 132.08) (end 104.255 130.429) (width 0.2) (layer "F.Cu") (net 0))
 (segment (start 92.837 80.391) (end 92.837 79.629) (width 0.2) (layer "F.Cu") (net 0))
 (segment (start 120.523 53.213) (end 120.65 53.34) (width 0.2) (layer "F.Cu") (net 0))
 (segment (start 78.613 63.5) (end 88.392 63.5) (width 0.2) (layer "F.Cu") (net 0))
 (segment (start 99.314 84.86) (end 100.69 84.86) (width 0.2) (layer "F.Cu") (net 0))
 (segment (start 97.917 98.933) (end 97.917 92.329) (width 0.6) (layer "F.Cu") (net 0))
 (segment (start 99.369 90.86) (end 98.806 90.297) (width 0.4) (layer "F.Cu") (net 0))
 (segment (start 85.11 131.465) (end 93.345 139.7) (width 0.6) (layer "F.Cu") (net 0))
 (segment (start 83.629 86.17) (end 82.564 86.17) (width 0.2) (layer "F.Cu") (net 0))
 (segment (start 99.672 92.86) (end 99.568 92.964) (width 0.2) (layer "F.Cu") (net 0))
 (segment (start 93.853 58.674) (end 93.853 55.626) (width 0.2) (layer "F.Cu") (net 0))
 (segment (start 104.43 119.09) (end 105.41 118.11) (width 0.2) (layer "F.Cu") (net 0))
 (segment (start 98.044 61.722) (end 95.885 59.563) (width 0.2) (layer "F.Cu") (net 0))
 (segment (start 90.805 131.445) (end 90.805 127) (width 0.6) (layer "F.Cu") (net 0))
 (segment (start 99.29 122.735) (end 95.315 126.71) (width 0.4) (layer "F.Cu") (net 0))
 (segment (start 103.759 129.921) (end 106.172 129.921) (width 0.2) (layer "F.Cu") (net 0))
 (segment (start 99.568 97.282) (end 102.108 99.822) (width 0.2) (layer "F.Cu") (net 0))
 (segment (start 103.265 119.09) (end 104.43 119.09) (width 0.2) (layer "F.Cu") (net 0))
 (segment (start 85.471 84.328) (end 83.629 86.17) (width 0.2) (layer "F.Cu") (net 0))
 (segment (start 117.348 55.935) (end 117.348 59.817) (width 0.2) (layer "F.Cu") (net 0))
 (segment (start 83.439 95.885) (end 90.17 89.154) (width 0.2) (layer "F.Cu") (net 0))
 (segment (start 80.391 65.278) (end 80.391 93.345) (width 0.2) (layer "F.Cu") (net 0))
 (segment (start 99.718 79.86) (end 98.655 80.923) (width 0.2) (layer "F.Cu") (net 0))
 (segment (start 90.17 104.14) (end 90.19 104.16) (width 0.6) (layer "F.Cu") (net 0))
 (segment (start 102.235 131.445) (end 103.759 129.921) (width 0.2) (layer "F.Cu") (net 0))
 (segment (start 78.613 63.5) (end 56.46 63.5) (width 0.2) (layer "F.Cu") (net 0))
 (segment (start 106.934 55.681) (end 105.99 54.737) (width 0.2) (layer "F.Cu") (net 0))
 (segment (start 85.757 92.17) (end 82.564 92.17) (width 0.2) (layer "F.Cu") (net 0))
 (segment (start 90.19 104.16) (end 90.19 106.075) (width 0.6) (layer "F.Cu") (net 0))
 (segment (start 104.775 130.937) (end 104.75 130.962) (width 0.2) (layer "F.Cu") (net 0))
 (segment (start 96.52 100.33) (end 92.71 104.14) (width 0.6) (layer "F.Cu") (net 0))
 (segment (start 94.742 59.563) (end 93.853 58.674) (width 0.2) (layer "F.Cu") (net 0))
 (segment (start 110.49 53.213) (end 110.49 54.737) (width 0.2) (layer "F.Cu") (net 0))
 (segment (start 89.535 88.392) (end 85.757 92.17) (width 0.2) (layer "F.Cu") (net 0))
 (segment (start 92.829 81.923) (end 91.331 81.923) (width 0.2) (layer "F.Cu") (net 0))
 (segment (start 92.71 104.14) (end 92.73 104.16) (width 0.6) (layer "F.Cu") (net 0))
 (segment (start 85.471 83.439) (end 85.471 84.328) (width 0.2) (layer "F.Cu") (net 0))
 (segment (start 102.108 99.822) (end 105.664 99.822) (width 0.2) (layer "F.Cu") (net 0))
 (segment (start 100.69 90.86) (end 99.369 90.86) (width 0.4) (layer "F.Cu") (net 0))
 (segment (start 81.407 89.662) (end 81.915 90.17) (width 0.2) (layer "F.Cu") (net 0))
 (segment (start 59.273 65.187) (end 71.918 65.187) (width 0.2) (layer "F.Cu") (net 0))
 (segment (start 97.917 91.186) (end 98.806 90.297) (width 0.6) (layer "F.Cu") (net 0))
 (segment (start 90.242 54.737) (end 91.766 53.213) (width 0.2) (layer "F.Cu") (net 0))
 (segment (start 105.41 100.838) (end 104.902 100.33) (width 0.2) (layer "F.Cu") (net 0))
 (segment (start 80.3275 65.2145) (end 78.613 63.5) (width 0.2) (layer "F.Cu") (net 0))
 (segment (start 95.885 59.563) (end 94.742 59.563) (width 0.2) (layer "F.Cu") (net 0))
 (segment (start 92.718 85.86) (end 100.69 85.86) (width 0.2) (layer "F.Cu") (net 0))
 (segment (start 98.806 88.392) (end 95.377 91.821) (width 0.6) (layer "F.Cu") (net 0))
 (segment (start 89.535 131.445) (end 89.535 127) (width 0.6) (layer "F.Cu") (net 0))
 (segment (start 100.69 89.86) (end 99.243 89.86) (width 0.4) (layer "F.Cu") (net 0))
 (segment (start 99.274 88.86) (end 98.806 88.392) (width 0.4) (layer "F.Cu") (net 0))
 (segment (start 78.994 72.263) (end 78.994 93.853) (width 0.2) (layer "F.Cu") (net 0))
 (segment (start 99.314 61.849) (end 99.314 79.375) (width 0.2) (layer "F.Cu") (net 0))
 (segment (start 104.902 100.33) (end 101.854 100.33) (width 0.2) (layer "F.Cu") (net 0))
 (segment (start 92.71 85.852) (end 92.718 85.86) (width 0.2) (layer "F.Cu") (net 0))
 (segment (start 88.106 88.17) (end 82.564 88.17) (width 0.2) (layer "F.Cu") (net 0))
 (segment (start 99.06 92.202) (end 99.402 91.86) (width 0.2) (layer "F.Cu") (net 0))
 (segment (start 99.568 92.964) (end 99.568 97.282) (width 0.2) (layer "F.Cu") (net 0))
 (segment (start 105.664 99.822) (end 106.68 100.838) (width 0.2) (layer "F.Cu") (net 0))
 (segment (start 106.172 130.937) (end 104.775 130.937) (width 0.2) (layer "F.Cu") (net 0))
 (segment (start 88.138 88.138) (end 88.106 88.17) (width 0.2) (layer "F.Cu") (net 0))
 (segment (start 81.026 95.885) (end 83.439 95.885) (width 0.2) (layer "F.Cu") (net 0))
 (via (at 92.71 89.154) (size 0.6) (drill 0.3) (layers "F.Cu" "B.Cu") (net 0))
 (via (at 99.314 84.86) (size 0.4) (drill 0.2) (layers "F.Cu" "B.Cu") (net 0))
 (via (at 89.535 131.445) (size 0.6) (drill 0.4) (layers "F.Cu" "B.Cu") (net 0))
 (via (at 92.71 85.852) (size 0.6) (drill 0.3) (layers "F.Cu" "B.Cu") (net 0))
 (via (at 97.79 130.175) (size 0.6) (drill 0.3) (layers "F.Cu" "B.Cu") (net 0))
 (via (at 104.75 130.962) (size 0.6) (drill 0.3) (layers "F.Cu" "B.Cu") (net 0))
 (via (at 102.096 132.715) (size 0.6) (drill 0.3) (layers "F.Cu" "B.Cu") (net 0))
 (via (at 103.112 132.715) (size 0.6) (drill 0.3) (layers "F.Cu" "B.Cu") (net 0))
 (via (at 85.471 83.439) (size 0.6) (drill 0.3) (layers "F.Cu" "B.Cu") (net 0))
 (via (at 100.838 130.175) (size 0.6) (drill 0.3) (layers "F.Cu" "B.Cu") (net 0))
 (via (at 98.044 79.375) (size 0.4) (drill 0.2) (layers "F.Cu" "B.Cu") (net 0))
 (via (at 85.471 81.915) (size 0.6) (drill 0.3) (layers "F.Cu" "B.Cu") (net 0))
 (via (at 88.138 88.138) (size 0.6) (drill 0.3) (layers "F.Cu" "B.Cu") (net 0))
 (via (at 98.679 79.375) (size 0.4) (drill 0.2) (layers "F.Cu" "B.Cu") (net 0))
 (via (at 89.40844 86.86756) (size 0.6) (drill 0.3) (layers "F.Cu" "B.Cu") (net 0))
 (via (at 89.535 127) (size 0.6) (drill 0.4) (layers "F.Cu" "B.Cu") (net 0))
 (via (at 99.314 79.375) (size 0.4) (drill 0.2) (layers "F.Cu" "B.Cu") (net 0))
 (via (at 90.805 127) (size 0.6) (drill 0.4) (layers "F.Cu" "B.Cu") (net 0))
 (via (at 92.837 80.391) (size 0.6) (drill 0.3) (layers "F.Cu" "B.Cu") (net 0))
 (via (at 98.044 82.86) (size 0.4) (drill 0.2) (layers "F.Cu" "B.Cu") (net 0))
 (via (at 102.235 131.445) (size 0.6) (drill 0.3) (layers "F.Cu" "B.Cu") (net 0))
 (via (at 98.679 83.86) (size 0.4) (drill 0.2) (layers "F.Cu" "B.Cu") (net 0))
 (via (at 92.837 81.915) (size 0.6) (drill 0.3) (layers "F.Cu" "B.Cu") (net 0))
 (via (at 104.775 129.413) (size 0.6) (drill 0.3) (layers "F.Cu" "B.Cu") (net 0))
 (via (at 90.805 131.445) (size 0.6) (drill 0.4) (layers "F.Cu" "B.Cu") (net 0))
 (segment (start 102.477 132.08) (end 102.6 132.203) (width 0.2) (layer "B.Cu") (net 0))
 (segment (start 80.03 125.75) (end 80.03 106.075) (width 0.6) (layer "B.Cu") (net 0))
 (segment (start 104.394 129.032) (end 99.187 129.032) (width 0.6) (layer "B.Cu") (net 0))
 (segment (start 102.235 131.445) (end 102.108 131.572) (width 0.2) (layer "B.Cu") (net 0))
 (segment (start 88.265 132.715) (end 89.535 131.445) (width 0.6) (layer "B.Cu") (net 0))
 (segment (start 99.95 131.063) (end 100.838 130.175) (width 0.6) (layer "B.Cu") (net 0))
 (segment (start 105.55 130.188) (end 105.55 134.07) (width 0.6) (layer "B.Cu") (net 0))
 (segment (start 102.1 132.719) (end 102.096 132.715) (width 0.2) (layer "B.Cu") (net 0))
 (segment (start 90.805 139.7) (end 90.805 131.445) (width 0.6) (layer "B.Cu") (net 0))
 (segment (start 101.6 132.195) (end 101.715 132.08) (width 0.2) (layer "B.Cu") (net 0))
 (segment (start 99.95 134.07) (end 99.95 131.063) (width 0.6) (layer "B.Cu") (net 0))
 (segment (start 101.6 134.07) (end 101.6 132.195) (width 0.2) (layer "B.Cu") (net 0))
 (segment (start 97.1425 107.315) (end 97.1625 107.335) (width 0.6) (layer "B.Cu") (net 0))
 (segment (start 93.98 108.585) (end 95.25 107.315) (width 0.6) (layer "B.Cu") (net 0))
 (segment (start 103.1 134.07) (end 103.1 132.727) (width 0.2) (layer "B.Cu") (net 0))
 (segment (start 102.1 134.07) (end 102.1 132.719) (width 0.2) (layer "B.Cu") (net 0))
 (segment (start 99.314 84.86) (end 99.314 79.375) (width 0.2) (layer "B.Cu") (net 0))
 (segment (start 89.535 109.855) (end 90.805 108.585) (width 0.6) (layer "B.Cu") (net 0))
 (segment (start 104.75 130.962) (end 104.75 134.07) (width 0.6) (layer "B.Cu") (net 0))
 (segment (start 89.40844 86.86756) (end 88.138 88.138) (width 0.2) (layer "B.Cu") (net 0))
 (segment (start 90.805 127) (end 90.805 113.665) (width 0.6) (layer "B.Cu") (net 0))
 (segment (start 82.57 125.75) (end 82.57 106.075) (width 0.6) (layer "B.Cu") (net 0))
 (segment (start 104.775 129.413) (end 104.394 129.032) (width 0.6) (layer "B.Cu") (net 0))
 (segment (start 102.096 132.08) (end 102.477 132.08) (width 0.2) (layer "B.Cu") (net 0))
 (segment (start 88.265 139.7) (end 88.265 132.715) (width 0.6) (layer "B.Cu") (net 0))
 (segment (start 102.6 132.203) (end 102.6 134.07) (width 0.2) (layer "B.Cu") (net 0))
 (segment (start 102.235 131.941) (end 102.235 131.445) (width 0.2) (layer "B.Cu") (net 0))
 (segment (start 90.805 108.585) (end 93.98 108.585) (width 0.6) (layer "B.Cu") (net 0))
 (segment (start 99.187 129.032) (end 98.806 128.651) (width 0.6) (layer "B.Cu") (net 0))
 (segment (start 85.471 128.651) (end 82.57 125.75) (width 0.6) (layer "B.Cu") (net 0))
 (segment (start 103.1 132.727) (end 103.112 132.715) (width 0.2) (layer "B.Cu") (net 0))
 (segment (start 101.715 132.08) (end 102.096 132.08) (width 0.2) (layer "B.Cu") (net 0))
 (segment (start 99.15 129.069) (end 99.15 134.07) (width 0.6) (layer "B.Cu") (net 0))
 (segment (start 92.837 81.915) (end 92.837 80.391) (width 0.2) (layer "B.Cu") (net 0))
 (segment (start 98.679 83.86) (end 98.679 79.375) (width 0.2) (layer "B.Cu") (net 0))
 (segment (start 90.805 113.665) (end 94.635 109.835) (width 0.6) (layer "B.Cu") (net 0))
 (segment (start 84.455 130.175) (end 80.03 125.75) (width 0.6) (layer "B.Cu") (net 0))
 (segment (start 94.635 109.835) (end 97.1625 109.835) (width 0.6) (layer "B.Cu") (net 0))
 (segment (start 89.535 127) (end 89.535 109.855) (width 0.6) (layer "B.Cu") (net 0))
 (segment (start 103.963 130.175) (end 104.75 130.962) (width 0.6) (layer "B.Cu") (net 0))
 (segment (start 89.36 113.76) (end 89.67 113.76) (width 0) (layer "B.Cu") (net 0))
 (segment (start 95.25 107.315) (end 97.1425 107.315) (width 0.6) (layer "B.Cu") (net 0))
 (segment (start 92.71 85.852) (end 92.71 89.154) (width 0.2) (layer "B.Cu") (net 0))
 (segment (start 104.775 129.413) (end 105.55 130.188) (width 0.6) (layer "B.Cu") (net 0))
 (segment (start 100.838 130.175) (end 100.458 130.555) (width 0.2) (layer "B.Cu") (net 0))
 (segment (start 100.838 130.175) (end 103.963 130.175) (width 0.6) (layer "B.Cu") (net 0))
 (segment (start 97.79 130.175) (end 84.455 130.175) (width 0.6) (layer "B.Cu") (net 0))
 (segment (start 98.044 82.86) (end 98.044 79.375) (width 0.2) (layer "B.Cu") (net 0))
 (segment (start 102.096 132.08) (end 102.235 131.941) (width 0.2) (layer "B.Cu") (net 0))
 (segment (start 98.806 128.651) (end 85.471 128.651) (width 0.6) (layer "B.Cu") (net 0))
 (segment (start 85.471 81.915) (end 85.471 83.439) (width 0.2) (layer "B.Cu") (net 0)))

